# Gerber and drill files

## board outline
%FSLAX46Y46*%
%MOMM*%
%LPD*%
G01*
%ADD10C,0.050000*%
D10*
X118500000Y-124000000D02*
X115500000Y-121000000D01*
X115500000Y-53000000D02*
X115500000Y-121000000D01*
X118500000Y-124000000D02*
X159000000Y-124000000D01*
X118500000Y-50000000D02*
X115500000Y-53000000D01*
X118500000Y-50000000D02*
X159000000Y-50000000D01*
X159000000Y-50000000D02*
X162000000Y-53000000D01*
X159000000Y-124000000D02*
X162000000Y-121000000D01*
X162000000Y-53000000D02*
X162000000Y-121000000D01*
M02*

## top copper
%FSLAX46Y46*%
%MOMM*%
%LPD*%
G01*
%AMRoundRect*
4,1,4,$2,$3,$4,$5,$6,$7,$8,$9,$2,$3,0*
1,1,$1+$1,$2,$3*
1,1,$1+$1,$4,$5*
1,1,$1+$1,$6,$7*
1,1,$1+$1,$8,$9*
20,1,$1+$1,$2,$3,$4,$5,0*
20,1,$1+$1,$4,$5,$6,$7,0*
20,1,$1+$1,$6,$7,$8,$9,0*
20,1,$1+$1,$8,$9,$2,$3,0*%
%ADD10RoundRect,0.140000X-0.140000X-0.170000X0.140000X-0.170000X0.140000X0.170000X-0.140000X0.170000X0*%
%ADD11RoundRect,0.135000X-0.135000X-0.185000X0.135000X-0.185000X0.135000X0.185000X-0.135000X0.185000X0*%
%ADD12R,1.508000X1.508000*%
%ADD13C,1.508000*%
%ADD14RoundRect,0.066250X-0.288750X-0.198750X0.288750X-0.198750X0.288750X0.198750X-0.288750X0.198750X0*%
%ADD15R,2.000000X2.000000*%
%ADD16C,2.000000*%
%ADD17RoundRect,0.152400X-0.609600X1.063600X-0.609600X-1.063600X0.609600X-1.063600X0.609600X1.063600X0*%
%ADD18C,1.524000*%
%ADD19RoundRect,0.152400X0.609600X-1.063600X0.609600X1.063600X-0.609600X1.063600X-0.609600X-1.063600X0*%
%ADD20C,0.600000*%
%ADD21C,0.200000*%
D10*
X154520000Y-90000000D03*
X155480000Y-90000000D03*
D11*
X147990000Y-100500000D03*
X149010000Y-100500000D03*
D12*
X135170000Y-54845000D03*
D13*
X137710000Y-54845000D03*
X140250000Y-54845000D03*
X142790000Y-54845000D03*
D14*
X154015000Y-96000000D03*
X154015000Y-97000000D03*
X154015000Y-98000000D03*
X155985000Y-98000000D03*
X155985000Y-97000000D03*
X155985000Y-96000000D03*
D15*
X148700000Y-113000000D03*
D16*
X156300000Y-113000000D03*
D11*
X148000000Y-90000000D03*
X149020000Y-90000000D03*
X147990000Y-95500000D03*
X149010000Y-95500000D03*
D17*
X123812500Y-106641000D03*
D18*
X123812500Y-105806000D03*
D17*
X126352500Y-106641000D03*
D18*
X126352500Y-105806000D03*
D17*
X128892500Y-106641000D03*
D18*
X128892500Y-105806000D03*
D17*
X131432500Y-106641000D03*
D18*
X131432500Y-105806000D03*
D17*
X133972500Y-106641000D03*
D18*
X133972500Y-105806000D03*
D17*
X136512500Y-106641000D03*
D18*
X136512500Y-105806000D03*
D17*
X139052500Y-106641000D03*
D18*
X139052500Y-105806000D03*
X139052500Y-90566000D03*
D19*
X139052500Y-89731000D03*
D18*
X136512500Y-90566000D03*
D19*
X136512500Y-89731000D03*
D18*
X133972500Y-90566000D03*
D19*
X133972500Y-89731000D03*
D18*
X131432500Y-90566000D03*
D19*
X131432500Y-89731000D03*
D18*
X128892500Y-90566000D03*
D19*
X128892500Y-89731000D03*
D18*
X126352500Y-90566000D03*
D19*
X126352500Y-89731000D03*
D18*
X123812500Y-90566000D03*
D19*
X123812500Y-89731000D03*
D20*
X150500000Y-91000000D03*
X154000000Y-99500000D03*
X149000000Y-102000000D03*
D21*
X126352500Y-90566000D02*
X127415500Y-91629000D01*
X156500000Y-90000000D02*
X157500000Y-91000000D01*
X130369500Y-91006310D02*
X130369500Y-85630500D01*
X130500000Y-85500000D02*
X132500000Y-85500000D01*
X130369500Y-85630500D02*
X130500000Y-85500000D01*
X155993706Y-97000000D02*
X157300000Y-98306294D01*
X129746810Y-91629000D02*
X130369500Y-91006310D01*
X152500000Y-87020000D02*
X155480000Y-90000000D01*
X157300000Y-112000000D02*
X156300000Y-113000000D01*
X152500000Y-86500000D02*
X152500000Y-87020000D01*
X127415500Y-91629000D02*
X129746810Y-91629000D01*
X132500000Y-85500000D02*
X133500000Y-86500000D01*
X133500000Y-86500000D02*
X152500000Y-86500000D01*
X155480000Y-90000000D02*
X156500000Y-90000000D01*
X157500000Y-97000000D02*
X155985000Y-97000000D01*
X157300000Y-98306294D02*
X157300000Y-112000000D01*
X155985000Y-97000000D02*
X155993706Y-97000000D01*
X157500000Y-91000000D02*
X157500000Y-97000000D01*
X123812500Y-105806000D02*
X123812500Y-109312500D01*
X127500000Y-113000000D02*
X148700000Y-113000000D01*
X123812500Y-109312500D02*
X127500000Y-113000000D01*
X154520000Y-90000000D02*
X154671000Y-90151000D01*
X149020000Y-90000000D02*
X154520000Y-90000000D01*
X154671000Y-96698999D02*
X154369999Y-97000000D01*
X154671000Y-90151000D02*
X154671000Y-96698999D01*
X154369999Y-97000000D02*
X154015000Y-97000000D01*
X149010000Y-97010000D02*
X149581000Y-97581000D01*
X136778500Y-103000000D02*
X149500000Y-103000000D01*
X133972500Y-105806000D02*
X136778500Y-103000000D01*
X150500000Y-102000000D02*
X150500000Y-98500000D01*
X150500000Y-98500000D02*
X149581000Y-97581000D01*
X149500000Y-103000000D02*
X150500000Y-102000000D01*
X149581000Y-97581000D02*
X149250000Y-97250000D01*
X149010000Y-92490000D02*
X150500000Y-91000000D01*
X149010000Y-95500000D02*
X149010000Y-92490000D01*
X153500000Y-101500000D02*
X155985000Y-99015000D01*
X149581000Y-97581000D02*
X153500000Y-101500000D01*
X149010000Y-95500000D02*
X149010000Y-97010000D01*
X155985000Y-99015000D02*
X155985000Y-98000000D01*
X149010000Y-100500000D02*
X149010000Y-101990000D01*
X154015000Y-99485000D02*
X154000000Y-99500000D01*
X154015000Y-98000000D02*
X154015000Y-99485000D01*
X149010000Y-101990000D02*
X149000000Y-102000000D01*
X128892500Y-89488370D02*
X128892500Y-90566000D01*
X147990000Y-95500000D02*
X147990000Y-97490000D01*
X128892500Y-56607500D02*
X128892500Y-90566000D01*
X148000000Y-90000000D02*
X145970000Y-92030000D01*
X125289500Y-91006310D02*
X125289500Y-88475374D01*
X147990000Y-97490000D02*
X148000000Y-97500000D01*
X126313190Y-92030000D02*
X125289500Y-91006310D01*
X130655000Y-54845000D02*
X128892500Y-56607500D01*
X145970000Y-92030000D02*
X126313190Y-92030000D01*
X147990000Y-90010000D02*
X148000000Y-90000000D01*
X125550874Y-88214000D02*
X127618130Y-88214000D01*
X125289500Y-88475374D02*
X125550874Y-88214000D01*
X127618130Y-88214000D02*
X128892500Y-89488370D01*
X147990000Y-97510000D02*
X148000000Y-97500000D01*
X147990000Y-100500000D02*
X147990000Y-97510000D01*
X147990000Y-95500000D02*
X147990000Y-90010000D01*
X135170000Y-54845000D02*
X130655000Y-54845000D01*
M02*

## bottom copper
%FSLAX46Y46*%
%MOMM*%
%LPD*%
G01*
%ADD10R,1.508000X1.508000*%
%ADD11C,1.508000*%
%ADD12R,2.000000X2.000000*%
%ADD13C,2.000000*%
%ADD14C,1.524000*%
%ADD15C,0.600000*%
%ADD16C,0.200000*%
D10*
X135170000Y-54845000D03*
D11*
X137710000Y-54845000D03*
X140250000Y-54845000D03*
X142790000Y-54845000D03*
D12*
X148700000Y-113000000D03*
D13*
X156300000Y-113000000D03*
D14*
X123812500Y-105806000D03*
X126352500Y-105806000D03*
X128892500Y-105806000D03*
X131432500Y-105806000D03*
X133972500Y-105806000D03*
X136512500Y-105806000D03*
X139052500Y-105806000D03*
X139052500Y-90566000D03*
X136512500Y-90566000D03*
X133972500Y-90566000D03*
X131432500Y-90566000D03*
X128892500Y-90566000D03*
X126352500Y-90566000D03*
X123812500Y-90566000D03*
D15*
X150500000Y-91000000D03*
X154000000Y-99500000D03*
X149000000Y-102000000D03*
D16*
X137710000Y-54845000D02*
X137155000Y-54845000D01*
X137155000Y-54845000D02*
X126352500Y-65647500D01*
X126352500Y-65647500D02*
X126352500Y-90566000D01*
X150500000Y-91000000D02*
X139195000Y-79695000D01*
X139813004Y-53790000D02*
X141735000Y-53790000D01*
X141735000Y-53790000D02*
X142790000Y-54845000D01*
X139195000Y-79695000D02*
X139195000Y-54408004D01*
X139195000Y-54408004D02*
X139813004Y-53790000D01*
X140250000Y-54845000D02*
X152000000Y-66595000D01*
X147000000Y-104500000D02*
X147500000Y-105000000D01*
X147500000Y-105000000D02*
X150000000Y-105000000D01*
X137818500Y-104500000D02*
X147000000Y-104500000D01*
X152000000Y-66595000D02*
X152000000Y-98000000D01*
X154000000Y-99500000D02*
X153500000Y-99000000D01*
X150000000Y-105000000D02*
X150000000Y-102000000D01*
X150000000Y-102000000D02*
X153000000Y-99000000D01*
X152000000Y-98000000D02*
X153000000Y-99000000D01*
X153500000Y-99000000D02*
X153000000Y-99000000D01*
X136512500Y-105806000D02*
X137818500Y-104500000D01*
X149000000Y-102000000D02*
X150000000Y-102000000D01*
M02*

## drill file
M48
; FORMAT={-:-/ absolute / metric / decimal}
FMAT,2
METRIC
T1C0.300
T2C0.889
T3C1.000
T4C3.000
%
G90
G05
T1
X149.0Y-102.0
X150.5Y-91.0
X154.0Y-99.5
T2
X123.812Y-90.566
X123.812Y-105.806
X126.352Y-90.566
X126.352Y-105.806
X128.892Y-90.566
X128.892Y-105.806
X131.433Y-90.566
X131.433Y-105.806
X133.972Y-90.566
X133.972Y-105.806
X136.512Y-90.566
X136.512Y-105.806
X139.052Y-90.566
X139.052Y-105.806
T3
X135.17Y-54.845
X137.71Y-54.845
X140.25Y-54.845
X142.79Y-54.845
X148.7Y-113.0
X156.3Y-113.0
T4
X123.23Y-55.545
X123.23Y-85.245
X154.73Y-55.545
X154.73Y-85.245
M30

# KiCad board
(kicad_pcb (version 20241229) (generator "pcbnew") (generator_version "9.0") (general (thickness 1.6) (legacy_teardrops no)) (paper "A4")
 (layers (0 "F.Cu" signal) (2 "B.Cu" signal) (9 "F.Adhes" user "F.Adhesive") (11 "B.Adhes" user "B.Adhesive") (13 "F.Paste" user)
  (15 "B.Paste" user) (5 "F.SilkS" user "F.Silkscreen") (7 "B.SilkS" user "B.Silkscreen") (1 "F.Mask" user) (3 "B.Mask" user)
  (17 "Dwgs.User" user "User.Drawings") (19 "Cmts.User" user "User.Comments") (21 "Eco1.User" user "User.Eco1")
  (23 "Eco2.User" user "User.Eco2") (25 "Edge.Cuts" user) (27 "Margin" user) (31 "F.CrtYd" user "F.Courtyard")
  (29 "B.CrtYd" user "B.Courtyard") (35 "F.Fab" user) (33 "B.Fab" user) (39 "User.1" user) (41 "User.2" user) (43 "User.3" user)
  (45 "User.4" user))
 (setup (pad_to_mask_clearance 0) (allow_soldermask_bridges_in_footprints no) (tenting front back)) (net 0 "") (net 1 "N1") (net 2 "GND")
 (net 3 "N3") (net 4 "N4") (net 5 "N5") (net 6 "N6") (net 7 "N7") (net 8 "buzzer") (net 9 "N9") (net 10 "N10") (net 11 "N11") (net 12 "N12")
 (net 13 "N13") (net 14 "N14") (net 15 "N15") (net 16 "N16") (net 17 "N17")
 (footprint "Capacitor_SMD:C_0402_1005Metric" (layer "F.Cu") (at 155 90)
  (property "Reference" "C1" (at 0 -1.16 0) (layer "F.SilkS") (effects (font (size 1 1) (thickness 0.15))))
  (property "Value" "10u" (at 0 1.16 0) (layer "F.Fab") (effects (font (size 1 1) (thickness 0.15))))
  (pad "1" smd roundrect (at -0.48 0) (size 0.56 0.62) (layers "F.Cu" "F.Mask" "F.Paste") (roundrect_rratio 0.25) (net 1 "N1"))
  (pad "2" smd roundrect (at 0.48 0) (size 0.56 0.62) (layers "F.Cu" "F.Mask" "F.Paste") (roundrect_rratio 0.25) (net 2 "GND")))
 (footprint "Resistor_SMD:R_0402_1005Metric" (layer "F.Cu") (at 148.5 100.5)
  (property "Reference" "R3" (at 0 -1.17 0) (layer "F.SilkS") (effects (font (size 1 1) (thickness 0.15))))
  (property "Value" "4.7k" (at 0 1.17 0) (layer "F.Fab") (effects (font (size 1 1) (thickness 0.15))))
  (pad "1" smd roundrect (at -0.51 0) (size 0.54 0.64) (layers "F.Cu" "F.Mask" "F.Paste") (roundrect_rratio 0.25) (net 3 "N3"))
  (pad "2" smd roundrect (at 0.51 0) (size 0.54 0.64) (layers "F.Cu" "F.Mask" "F.Paste") (roundrect_rratio 0.25) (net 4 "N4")))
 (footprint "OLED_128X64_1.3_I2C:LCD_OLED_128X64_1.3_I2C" (layer "F.Cu") (at 138.98 70.395)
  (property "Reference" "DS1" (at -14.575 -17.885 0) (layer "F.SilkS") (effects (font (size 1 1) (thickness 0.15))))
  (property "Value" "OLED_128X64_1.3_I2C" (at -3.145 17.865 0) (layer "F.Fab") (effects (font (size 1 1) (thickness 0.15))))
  (pad "" np_thru_hole circle (at -15.75 -14.85) (size 3 3) (drill 3) (layers "*.Cu" "*.Mask"))
  (pad "" np_thru_hole circle (at -15.75 14.85) (size 3 3) (drill 3) (layers "*.Cu" "*.Mask"))
  (pad "" np_thru_hole circle (at 15.75 -14.85) (size 3 3) (drill 3) (layers "*.Cu" "*.Mask"))
  (pad "" np_thru_hole circle (at 15.75 14.85) (size 3 3) (drill 3) (layers "*.Cu" "*.Mask"))
  (pad "1" thru_hole rect (at -3.81 -15.55) (size 1.508 1.508) (drill 1) (layers "*.Cu" "*.Mask") (remove_unused_layers no) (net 3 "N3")
   (solder_mask_margin 0.102))
  (pad "2" thru_hole circle (at -1.27 -15.55) (size 1.508 1.508) (drill 1) (layers "*.Cu" "*.Mask") (remove_unused_layers no) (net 2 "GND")
   (solder_mask_margin 0.102))
  (pad "3" thru_hole circle (at 1.27 -15.55) (size 1.508 1.508) (drill 1) (layers "*.Cu" "*.Mask") (remove_unused_layers no) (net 4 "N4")
   (solder_mask_margin 0.102))
  (pad "4" thru_hole circle (at 3.81 -15.55) (size 1.508 1.508) (drill 1) (layers "*.Cu" "*.Mask") (remove_unused_layers no) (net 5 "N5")
   (solder_mask_margin 0.102)))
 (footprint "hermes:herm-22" (layer "F.Cu") (at 124 115.5)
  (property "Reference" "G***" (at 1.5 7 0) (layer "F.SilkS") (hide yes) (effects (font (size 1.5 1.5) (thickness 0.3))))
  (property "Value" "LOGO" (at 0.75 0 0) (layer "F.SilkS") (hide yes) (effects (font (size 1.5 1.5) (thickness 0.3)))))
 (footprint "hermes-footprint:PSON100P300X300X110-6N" (layer "F.Cu") (at 155 97)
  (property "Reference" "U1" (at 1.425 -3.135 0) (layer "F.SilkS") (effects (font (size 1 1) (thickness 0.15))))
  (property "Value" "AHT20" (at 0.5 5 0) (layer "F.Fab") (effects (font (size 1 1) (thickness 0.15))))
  (pad "1" smd roundrect (at -0.985 -1) (size 0.71 0.53) (layers "F.Cu" "F.Mask" "F.Paste") (roundrect_rratio 0.125) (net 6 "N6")
   (solder_mask_margin 0.102))
  (pad "2" smd roundrect (at -0.985 0) (size 0.71 0.53) (layers "F.Cu" "F.Mask" "F.Paste") (roundrect_rratio 0.125) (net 1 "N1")
   (solder_mask_margin 0.102))
  (pad "3" smd roundrect (at -0.985 1) (size 0.71 0.53) (layers "F.Cu" "F.Mask" "F.Paste") (roundrect_rratio 0.125) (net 4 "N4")
   (solder_mask_margin 0.102))
  (pad "4" smd roundrect (at 0.985 1) (size 0.71 0.53) (layers "F.Cu" "F.Mask" "F.Paste") (roundrect_rratio 0.125) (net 5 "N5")
   (solder_mask_margin 0.102))
  (pad "5" smd roundrect (at 0.985 0) (size 0.71 0.53) (layers "F.Cu" "F.Mask" "F.Paste") (roundrect_rratio 0.125) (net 2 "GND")
   (solder_mask_margin 0.102))
  (pad "6" smd roundrect (at 0.985 -1) (size 0.71 0.53) (layers "F.Cu" "F.Mask" "F.Paste") (roundrect_rratio 0.125) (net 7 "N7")
   (solder_mask_margin 0.102)))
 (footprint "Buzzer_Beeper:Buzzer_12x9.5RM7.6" (layer "F.Cu") (at 148.7 113)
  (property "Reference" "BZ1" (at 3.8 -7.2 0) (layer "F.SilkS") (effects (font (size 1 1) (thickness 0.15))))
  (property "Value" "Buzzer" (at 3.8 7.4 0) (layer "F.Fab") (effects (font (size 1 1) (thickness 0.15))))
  (pad "1" thru_hole rect (at 0 0) (size 2 2) (drill 1) (layers "*.Cu" "*.Mask") (remove_unused_layers no) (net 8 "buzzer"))
  (pad "2" thru_hole circle (at 7.6 0) (size 2 2) (drill 1) (layers "*.Cu" "*.Mask") (remove_unused_layers no) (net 2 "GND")))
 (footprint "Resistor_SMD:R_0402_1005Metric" (layer "F.Cu") (at 148.51 90)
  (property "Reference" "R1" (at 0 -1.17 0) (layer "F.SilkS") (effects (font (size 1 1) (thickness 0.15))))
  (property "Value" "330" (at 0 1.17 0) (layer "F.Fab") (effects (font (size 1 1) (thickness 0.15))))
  (pad "1" smd roundrect (at -0.51 0) (size 0.54 0.64) (layers "F.Cu" "F.Mask" "F.Paste") (roundrect_rratio 0.25) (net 3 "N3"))
  (pad "2" smd roundrect (at 0.51 0) (size 0.54 0.64) (layers "F.Cu" "F.Mask" "F.Paste") (roundrect_rratio 0.25) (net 1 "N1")))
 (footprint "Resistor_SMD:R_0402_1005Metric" (layer "F.Cu") (at 148.5 95.5)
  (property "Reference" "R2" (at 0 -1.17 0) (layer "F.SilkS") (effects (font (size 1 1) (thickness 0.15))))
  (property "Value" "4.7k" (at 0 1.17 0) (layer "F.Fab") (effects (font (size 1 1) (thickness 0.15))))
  (pad "1" smd roundrect (at -0.51 0) (size 0.54 0.64) (layers "F.Cu" "F.Mask" "F.Paste") (roundrect_rratio 0.25) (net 3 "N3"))
  (pad "2" smd roundrect (at 0.51 0) (size 0.54 0.64) (layers "F.Cu" "F.Mask" "F.Paste") (roundrect_rratio 0.25) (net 5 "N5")))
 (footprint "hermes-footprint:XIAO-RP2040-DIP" (layer "F.Cu") (at 131.4325 98.186 180)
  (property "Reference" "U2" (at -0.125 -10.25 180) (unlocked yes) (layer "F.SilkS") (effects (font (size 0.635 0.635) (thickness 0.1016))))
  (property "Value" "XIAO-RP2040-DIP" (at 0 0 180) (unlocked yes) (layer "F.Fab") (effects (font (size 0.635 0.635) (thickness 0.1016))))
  (pad "1" smd roundrect (at 7.62 -8.455 270) (size 2.432 1.524) (layers "F.Cu" "F.Mask") (roundrect_rratio 0.1) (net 8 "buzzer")
   (thermal_bridge_angle 45))
  (pad "1" thru_hole circle (at 7.62 -7.62 270) (size 1.524 1.524) (drill 0.889) (layers "*.Cu" "*.Mask") (remove_unused_layers no)
   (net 8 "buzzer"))
  (pad "2" smd roundrect (at 5.08 -8.455 270) (size 2.432 1.524) (layers "F.Cu" "F.Mask") (roundrect_rratio 0.1) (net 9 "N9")
   (thermal_bridge_angle 45))
  (pad "2" thru_hole circle (at 5.08 -7.62 270) (size 1.524 1.524) (drill 0.889) (layers "*.Cu" "*.Mask") (remove_unused_layers no)
   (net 9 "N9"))
  (pad "3" smd roundrect (at 2.54 -8.455 270) (size 2.432 1.524) (layers "F.Cu" "F.Mask") (roundrect_rratio 0.1) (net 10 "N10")
   (thermal_bridge_angle 45))
  (pad "3" thru_hole circle (at 2.54 -7.62 270) (size 1.524 1.524) (drill 0.889) (layers "*.Cu" "*.Mask") (remove_unused_layers no)
   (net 10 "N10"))
  (pad "4" smd roundrect (at 0 -8.455 270) (size 2.432 1.524) (layers "F.Cu" "F.Mask") (roundrect_rratio 0.1) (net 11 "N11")
   (thermal_bridge_angle 45))
  (pad "4" thru_hole circle (at 0 -7.62 270) (size 1.524 1.524) (drill 0.889) (layers "*.Cu" "*.Mask") (remove_unused_layers no)
   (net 11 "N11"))
  (pad "5" smd roundrect (at -2.54 -8.455 270) (size 2.432 1.524) (layers "F.Cu" "F.Mask") (roundrect_rratio 0.1) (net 5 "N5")
   (thermal_bridge_angle 45))
  (pad "5" thru_hole circle (at -2.54 -7.62 270) (size 1.524 1.524) (drill 0.889) (layers "*.Cu" "*.Mask") (remove_unused_layers no)
   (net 5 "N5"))
  (pad "6" smd roundrect (at -5.08 -8.455 270) (size 2.432 1.524) (layers "F.Cu" "F.Mask") (roundrect_rratio 0.1) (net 4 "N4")
   (thermal_bridge_angle 45))
  (pad "6" thru_hole circle (at -5.08 -7.62 270) (size 1.524 1.524) (drill 0.889) (layers "*.Cu" "*.Mask") (remove_unused_layers no)
   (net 4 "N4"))
  (pad "7" smd roundrect (at -7.62 -8.455 270) (size 2.432 1.524) (layers "F.Cu" "F.Mask") (roundrect_rratio 0.1) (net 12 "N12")
   (thermal_bridge_angle 45))
  (pad "7" thru_hole circle (at -7.62 -7.62 270) (size 1.524 1.524) (drill 0.889) (layers "*.Cu" "*.Mask") (remove_unused_layers no)
   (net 12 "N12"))
  (pad "8" thru_hole circle (at -7.62 7.62 90) (size 1.524 1.524) (drill 0.889) (layers "*.Cu" "*.Mask") (remove_unused_layers no)
   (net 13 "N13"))
  (pad "8" smd roundrect (at -7.62 8.455 90) (size 2.432 1.524) (layers "F.Cu" "F.Mask") (roundrect_rratio 0.1) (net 13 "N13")
   (thermal_bridge_angle 45))
  (pad "9" thru_hole circle (at -5.08 7.62 90) (size 1.524 1.524) (drill 0.889) (layers "*.Cu" "*.Mask") (remove_unused_layers no)
   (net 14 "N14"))
  (pad "9" smd roundrect (at -5.08 8.455 90) (size 2.432 1.524) (layers "F.Cu" "F.Mask") (roundrect_rratio 0.1) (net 14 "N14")
   (thermal_bridge_angle 45))
  (pad "10" thru_hole circle (at -2.54 7.62 90) (size 1.524 1.524) (drill 0.889) (layers "*.Cu" "*.Mask") (remove_unused_layers no)
   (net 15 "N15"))
  (pad "10" smd roundrect (at -2.54 8.455 90) (size 2.432 1.524) (layers "F.Cu" "F.Mask") (roundrect_rratio 0.1) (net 15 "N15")
   (thermal_bridge_angle 45))
  (pad "11" thru_hole circle (at 0 7.62 90) (size 1.524 1.524) (drill 0.889) (layers "*.Cu" "*.Mask") (remove_unused_layers no)
   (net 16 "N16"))
  (pad "11" smd roundrect (at 0 8.455 90) (size 2.432 1.524) (layers "F.Cu" "F.Mask") (roundrect_rratio 0.1) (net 16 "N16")
   (thermal_bridge_angle 45))
  (pad "12" thru_hole circle (at 2.54 7.62 90) (size 1.524 1.524) (drill 0.889) (layers "*.Cu" "*.Mask") (remove_unused_layers no)
   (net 3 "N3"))
  (pad "12" smd roundrect (at 2.54 8.455 90) (size 2.432 1.524) (layers "F.Cu" "F.Mask") (roundrect_rratio 0.1) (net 3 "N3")
   (thermal_bridge_angle 45))
  (pad "13" thru_hole circle (at 5.08 7.62 90) (size 1.524 1.524) (drill 0.889) (layers "*.Cu" "*.Mask") (remove_unused_layers no)
   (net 2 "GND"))
  (pad "13" smd roundrect (at 5.08 8.455 90) (size 2.432 1.524) (layers "F.Cu" "F.Mask") (roundrect_rratio 0.1) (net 2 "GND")
   (thermal_bridge_angle 45))
  (pad "14" thru_hole circle (at 7.62 7.62 90) (size 1.524 1.524) (drill 0.889) (layers "*.Cu" "*.Mask") (remove_unused_layers no)
   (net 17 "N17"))
  (pad "14" smd roundrect (at 7.62 8.455 90) (size 2.432 1.524) (layers "F.Cu" "F.Mask") (roundrect_rratio 0.1) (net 17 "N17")
   (thermal_bridge_angle 45)))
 (gr_line (start 118.5 124) (end 115.5 121) (stroke (width 0.05) (type default)) (layer "Edge.Cuts"))
 (gr_line (start 115.5 53) (end 115.5 121) (stroke (width 0.05) (type default)) (layer "Edge.Cuts"))
 (gr_line (start 118.5 124) (end 159 124) (stroke (width 0.05) (type default)) (layer "Edge.Cuts"))
 (gr_line (start 118.5 50) (end 115.5 53) (stroke (width 0.05) (type default)) (layer "Edge.Cuts"))
 (gr_line (start 118.5 50) (end 159 50) (stroke (width 0.05) (type default)) (layer "Edge.Cuts"))
 (gr_line (start 159 50) (end 162 53) (stroke (width 0.05) (type default)) (layer "Edge.Cuts"))
 (gr_line (start 159 124) (end 162 121) (stroke (width 0.05) (type default)) (layer "Edge.Cuts"))
 (gr_line (start 162 53) (end 162 121) (stroke (width 0.05) (type default)) (layer "Edge.Cuts"))
 (segment (start 126.3525 90.566) (end 127.4155 91.629) (width 0.2) (layer "F.Cu") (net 2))
 (segment (start 156.5 90) (end 157.5 91) (width 0.2) (layer "F.Cu") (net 2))
 (segment (start 130.3695 91.00631) (end 130.3695 85.6305) (width 0.2) (layer "F.Cu") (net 2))
 (segment (start 130.5 85.5) (end 132.5 85.5) (width 0.2) (layer "F.Cu") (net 2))
 (segment (start 130.3695 85.6305) (end 130.5 85.5) (width 0.2) (layer "F.Cu") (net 2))
 (segment (start 155.993706 97) (end 157.3 98.306294) (width 0.2) (layer "F.Cu") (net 2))
 (segment (start 129.74681 91.629) (end 130.3695 91.00631) (width 0.2) (layer "F.Cu") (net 2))
 (segment (start 152.5 87.02) (end 155.48 90) (width 0.2) (layer "F.Cu") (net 2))
 (segment (start 157.3 112) (end 156.3 113) (width 0.2) (layer "F.Cu") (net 2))
 (segment (start 152.5 86.5) (end 152.5 87.02) (width 0.2) (layer "F.Cu") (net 2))
 (segment (start 127.4155 91.629) (end 129.74681 91.629) (width 0.2) (layer "F.Cu") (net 2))
 (segment (start 132.5 85.5) (end 133.5 86.5) (width 0.2) (layer "F.Cu") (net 2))
 (segment (start 133.5 86.5) (end 152.5 86.5) (width 0.2) (layer "F.Cu") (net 2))
 (segment (start 155.48 90) (end 156.5 90) (width 0.2) (layer "F.Cu") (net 2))
 (segment (start 157.5 97) (end 155.985 97) (width 0.2) (layer "F.Cu") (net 2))
 (segment (start 157.3 98.306294) (end 157.3 112) (width 0.2) (layer "F.Cu") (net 2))
 (segment (start 155.985 97) (end 155.993706 97) (width 0.2) (layer "F.Cu") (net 2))
 (segment (start 157.5 91) (end 157.5 97) (width 0.2) (layer "F.Cu") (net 2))
 (segment (start 137.71 54.845) (end 137.155 54.845) (width 0.2) (layer "B.Cu") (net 2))
 (segment (start 137.155 54.845) (end 126.3525 65.6475) (width 0.2) (layer "B.Cu") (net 2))
 (segment (start 126.3525 65.6475) (end 126.3525 90.566) (width 0.2) (layer "B.Cu") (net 2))
 (segment (start 123.8125 105.806) (end 123.8125 109.3125) (width 0.2) (layer "F.Cu") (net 8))
 (segment (start 127.5 113) (end 148.7 113) (width 0.2) (layer "F.Cu") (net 8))
 (segment (start 123.8125 109.3125) (end 127.5 113) (width 0.2) (layer "F.Cu") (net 8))
 (segment (start 154.52 90) (end 154.671 90.151) (width 0.2) (layer "F.Cu") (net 1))
 (segment (start 149.02 90) (end 154.52 90) (width 0.2) (layer "F.Cu") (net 1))
 (segment (start 154.671 96.698999) (end 154.369999 97) (width 0.2) (layer "F.Cu") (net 1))
 (segment (start 154.671 90.151) (end 154.671 96.698999) (width 0.2) (layer "F.Cu") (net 1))
 (segment (start 154.369999 97) (end 154.015 97) (width 0.2) (layer "F.Cu") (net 1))
 (segment (start 149.01 97.01) (end 149.581 97.581) (width 0.2) (layer "F.Cu") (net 5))
 (segment (start 136.7785 103) (end 149.5 103) (width 0.2) (layer "F.Cu") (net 5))
 (segment (start 133.9725 105.806) (end 136.7785 103) (width 0.2) (layer "F.Cu") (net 5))
 (segment (start 150.5 102) (end 150.5 98.5) (width 0.2) (layer "F.Cu") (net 5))
 (segment (start 150.5 98.5) (end 149.581 97.581) (width 0.2) (layer "F.Cu") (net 5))
 (segment (start 149.5 103) (end 150.5 102) (width 0.2) (layer "F.Cu") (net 5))
 (segment (start 149.581 97.581) (end 149.25 97.25) (width 0.2) (layer "F.Cu") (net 5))
 (segment (start 149.01 92.49) (end 150.5 91) (width 0.2) (layer "F.Cu") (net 5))
 (segment (start 149.01 95.5) (end 149.01 92.49) (width 0.2) (layer "F.Cu") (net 5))
 (segment (start 153.5 101.5) (end 155.985 99.015) (width 0.2) (layer "F.Cu") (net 5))
 (segment (start 149.581 97.581) (end 153.5 101.5) (width 0.2) (layer "F.Cu") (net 5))
 (segment (start 149.01 95.5) (end 149.01 97.01) (width 0.2) (layer "F.Cu") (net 5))
 (segment (start 155.985 99.015) (end 155.985 98) (width 0.2) (layer "F.Cu") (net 5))
 (via (at 150.5 91) (size 0.6) (drill 0.3) (layers "F.Cu" "B.Cu") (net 5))
 (segment (start 150.5 91) (end 139.195 79.695) (width 0.2) (layer "B.Cu") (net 5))
 (segment (start 139.813004 53.79) (end 141.735 53.79) (width 0.2) (layer "B.Cu") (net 5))
 (segment (start 141.735 53.79) (end 142.79 54.845) (width 0.2) (layer "B.Cu") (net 5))
 (segment (start 139.195 79.695) (end 139.195 54.408004) (width 0.2) (layer "B.Cu") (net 5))
 (segment (start 139.195 54.408004) (end 139.813004 53.79) (width 0.2) (layer "B.Cu") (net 5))
 (segment (start 149.01 100.5) (end 149.01 101.99) (width 0.2) (layer "F.Cu") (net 4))
 (segment (start 154.015 99.485) (end 154 99.5) (width 0.2) (layer "F.Cu") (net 4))
 (segment (start 154.015 98) (end 154.015 99.485) (width 0.2) (layer "F.Cu") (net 4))
 (segment (start 149.01 101.99) (end 149 102) (width 0.2) (layer "F.Cu") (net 4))
 (via (at 154 99.5) (size 0.6) (drill 0.3) (layers "F.Cu" "B.Cu") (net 4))
 (via (at 149 102) (size 0.6) (drill 0.3) (layers "F.Cu" "B.Cu") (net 4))
 (segment (start 140.25 54.845) (end 152 66.595) (width 0.2) (layer "B.Cu") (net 4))
 (segment (start 147 104.5) (end 147.5 105) (width 0.2) (layer "B.Cu") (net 4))
 (segment (start 147.5 105) (end 150 105) (width 0.2) (layer "B.Cu") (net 4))
 (segment (start 137.8185 104.5) (end 147 104.5) (width 0.2) (layer "B.Cu") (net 4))
 (segment (start 152 66.595) (end 152 98) (width 0.2) (layer "B.Cu") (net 4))
 (segment (start 154 99.5) (end 153.5 99) (width 0.2) (layer "B.Cu") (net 4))
 (segment (start 150 105) (end 150 102) (width 0.2) (layer "B.Cu") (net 4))
 (segment (start 150 102) (end 153 99) (width 0.2) (layer "B.Cu") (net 4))
 (segment (start 152 98) (end 153 99) (width 0.2) (layer "B.Cu") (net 4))
 (segment (start 153.5 99) (end 153 99) (width 0.2) (layer "B.Cu") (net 4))
 (segment (start 136.5125 105.806) (end 137.8185 104.5) (width 0.2) (layer "B.Cu") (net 4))
 (segment (start 149 102) (end 150 102) (width 0.2) (layer "B.Cu") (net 4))
 (segment (start 128.8925 89.48837) (end 128.8925 90.566) (width 0.2) (layer "F.Cu") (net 3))
 (segment (start 147.99 95.5) (end 147.99 97.49) (width 0.2) (layer "F.Cu") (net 3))
 (segment (start 128.8925 56.6075) (end 128.8925 90.566) (width 0.2) (layer "F.Cu") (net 3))
 (segment (start 148 90) (end 145.97 92.03) (width 0.2) (layer "F.Cu") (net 3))
 (segment (start 125.2895 91.00631) (end 125.2895 88.475374) (width 0.2) (layer "F.Cu") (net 3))
 (segment (start 147.99 97.49) (end 148 97.5) (width 0.2) (layer "F.Cu") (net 3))
 (segment (start 126.31319 92.03) (end 125.2895 91.00631) (width 0.2) (layer "F.Cu") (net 3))
 (segment (start 130.655 54.845) (end 128.8925 56.6075) (width 0.2) (layer "F.Cu") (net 3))
 (segment (start 145.97 92.03) (end 126.31319 92.03) (width 0.2) (layer "F.Cu") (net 3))
 (segment (start 147.99 90.01) (end 148 90) (width 0.2) (layer "F.Cu") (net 3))
 (segment (start 125.550874 88.214) (end 127.61813 88.214) (width 0.2) (layer "F.Cu") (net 3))
 (segment (start 125.2895 88.475374) (end 125.550874 88.214) (width 0.2) (layer "F.Cu") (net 3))
 (segment (start 127.61813 88.214) (end 128.8925 89.48837) (width 0.2) (layer "F.Cu") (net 3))
 (segment (start 147.99 97.51) (end 148 97.5) (width 0.2) (layer "F.Cu") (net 3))
 (segment (start 147.99 100.5) (end 147.99 97.51) (width 0.2) (layer "F.Cu") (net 3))
 (segment (start 147.99 95.5) (end 147.99 90.01) (width 0.2) (layer "F.Cu") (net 3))
 (segment (start 135.17 54.845) (end 130.655 54.845) (width 0.2) (layer "F.Cu") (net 3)))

